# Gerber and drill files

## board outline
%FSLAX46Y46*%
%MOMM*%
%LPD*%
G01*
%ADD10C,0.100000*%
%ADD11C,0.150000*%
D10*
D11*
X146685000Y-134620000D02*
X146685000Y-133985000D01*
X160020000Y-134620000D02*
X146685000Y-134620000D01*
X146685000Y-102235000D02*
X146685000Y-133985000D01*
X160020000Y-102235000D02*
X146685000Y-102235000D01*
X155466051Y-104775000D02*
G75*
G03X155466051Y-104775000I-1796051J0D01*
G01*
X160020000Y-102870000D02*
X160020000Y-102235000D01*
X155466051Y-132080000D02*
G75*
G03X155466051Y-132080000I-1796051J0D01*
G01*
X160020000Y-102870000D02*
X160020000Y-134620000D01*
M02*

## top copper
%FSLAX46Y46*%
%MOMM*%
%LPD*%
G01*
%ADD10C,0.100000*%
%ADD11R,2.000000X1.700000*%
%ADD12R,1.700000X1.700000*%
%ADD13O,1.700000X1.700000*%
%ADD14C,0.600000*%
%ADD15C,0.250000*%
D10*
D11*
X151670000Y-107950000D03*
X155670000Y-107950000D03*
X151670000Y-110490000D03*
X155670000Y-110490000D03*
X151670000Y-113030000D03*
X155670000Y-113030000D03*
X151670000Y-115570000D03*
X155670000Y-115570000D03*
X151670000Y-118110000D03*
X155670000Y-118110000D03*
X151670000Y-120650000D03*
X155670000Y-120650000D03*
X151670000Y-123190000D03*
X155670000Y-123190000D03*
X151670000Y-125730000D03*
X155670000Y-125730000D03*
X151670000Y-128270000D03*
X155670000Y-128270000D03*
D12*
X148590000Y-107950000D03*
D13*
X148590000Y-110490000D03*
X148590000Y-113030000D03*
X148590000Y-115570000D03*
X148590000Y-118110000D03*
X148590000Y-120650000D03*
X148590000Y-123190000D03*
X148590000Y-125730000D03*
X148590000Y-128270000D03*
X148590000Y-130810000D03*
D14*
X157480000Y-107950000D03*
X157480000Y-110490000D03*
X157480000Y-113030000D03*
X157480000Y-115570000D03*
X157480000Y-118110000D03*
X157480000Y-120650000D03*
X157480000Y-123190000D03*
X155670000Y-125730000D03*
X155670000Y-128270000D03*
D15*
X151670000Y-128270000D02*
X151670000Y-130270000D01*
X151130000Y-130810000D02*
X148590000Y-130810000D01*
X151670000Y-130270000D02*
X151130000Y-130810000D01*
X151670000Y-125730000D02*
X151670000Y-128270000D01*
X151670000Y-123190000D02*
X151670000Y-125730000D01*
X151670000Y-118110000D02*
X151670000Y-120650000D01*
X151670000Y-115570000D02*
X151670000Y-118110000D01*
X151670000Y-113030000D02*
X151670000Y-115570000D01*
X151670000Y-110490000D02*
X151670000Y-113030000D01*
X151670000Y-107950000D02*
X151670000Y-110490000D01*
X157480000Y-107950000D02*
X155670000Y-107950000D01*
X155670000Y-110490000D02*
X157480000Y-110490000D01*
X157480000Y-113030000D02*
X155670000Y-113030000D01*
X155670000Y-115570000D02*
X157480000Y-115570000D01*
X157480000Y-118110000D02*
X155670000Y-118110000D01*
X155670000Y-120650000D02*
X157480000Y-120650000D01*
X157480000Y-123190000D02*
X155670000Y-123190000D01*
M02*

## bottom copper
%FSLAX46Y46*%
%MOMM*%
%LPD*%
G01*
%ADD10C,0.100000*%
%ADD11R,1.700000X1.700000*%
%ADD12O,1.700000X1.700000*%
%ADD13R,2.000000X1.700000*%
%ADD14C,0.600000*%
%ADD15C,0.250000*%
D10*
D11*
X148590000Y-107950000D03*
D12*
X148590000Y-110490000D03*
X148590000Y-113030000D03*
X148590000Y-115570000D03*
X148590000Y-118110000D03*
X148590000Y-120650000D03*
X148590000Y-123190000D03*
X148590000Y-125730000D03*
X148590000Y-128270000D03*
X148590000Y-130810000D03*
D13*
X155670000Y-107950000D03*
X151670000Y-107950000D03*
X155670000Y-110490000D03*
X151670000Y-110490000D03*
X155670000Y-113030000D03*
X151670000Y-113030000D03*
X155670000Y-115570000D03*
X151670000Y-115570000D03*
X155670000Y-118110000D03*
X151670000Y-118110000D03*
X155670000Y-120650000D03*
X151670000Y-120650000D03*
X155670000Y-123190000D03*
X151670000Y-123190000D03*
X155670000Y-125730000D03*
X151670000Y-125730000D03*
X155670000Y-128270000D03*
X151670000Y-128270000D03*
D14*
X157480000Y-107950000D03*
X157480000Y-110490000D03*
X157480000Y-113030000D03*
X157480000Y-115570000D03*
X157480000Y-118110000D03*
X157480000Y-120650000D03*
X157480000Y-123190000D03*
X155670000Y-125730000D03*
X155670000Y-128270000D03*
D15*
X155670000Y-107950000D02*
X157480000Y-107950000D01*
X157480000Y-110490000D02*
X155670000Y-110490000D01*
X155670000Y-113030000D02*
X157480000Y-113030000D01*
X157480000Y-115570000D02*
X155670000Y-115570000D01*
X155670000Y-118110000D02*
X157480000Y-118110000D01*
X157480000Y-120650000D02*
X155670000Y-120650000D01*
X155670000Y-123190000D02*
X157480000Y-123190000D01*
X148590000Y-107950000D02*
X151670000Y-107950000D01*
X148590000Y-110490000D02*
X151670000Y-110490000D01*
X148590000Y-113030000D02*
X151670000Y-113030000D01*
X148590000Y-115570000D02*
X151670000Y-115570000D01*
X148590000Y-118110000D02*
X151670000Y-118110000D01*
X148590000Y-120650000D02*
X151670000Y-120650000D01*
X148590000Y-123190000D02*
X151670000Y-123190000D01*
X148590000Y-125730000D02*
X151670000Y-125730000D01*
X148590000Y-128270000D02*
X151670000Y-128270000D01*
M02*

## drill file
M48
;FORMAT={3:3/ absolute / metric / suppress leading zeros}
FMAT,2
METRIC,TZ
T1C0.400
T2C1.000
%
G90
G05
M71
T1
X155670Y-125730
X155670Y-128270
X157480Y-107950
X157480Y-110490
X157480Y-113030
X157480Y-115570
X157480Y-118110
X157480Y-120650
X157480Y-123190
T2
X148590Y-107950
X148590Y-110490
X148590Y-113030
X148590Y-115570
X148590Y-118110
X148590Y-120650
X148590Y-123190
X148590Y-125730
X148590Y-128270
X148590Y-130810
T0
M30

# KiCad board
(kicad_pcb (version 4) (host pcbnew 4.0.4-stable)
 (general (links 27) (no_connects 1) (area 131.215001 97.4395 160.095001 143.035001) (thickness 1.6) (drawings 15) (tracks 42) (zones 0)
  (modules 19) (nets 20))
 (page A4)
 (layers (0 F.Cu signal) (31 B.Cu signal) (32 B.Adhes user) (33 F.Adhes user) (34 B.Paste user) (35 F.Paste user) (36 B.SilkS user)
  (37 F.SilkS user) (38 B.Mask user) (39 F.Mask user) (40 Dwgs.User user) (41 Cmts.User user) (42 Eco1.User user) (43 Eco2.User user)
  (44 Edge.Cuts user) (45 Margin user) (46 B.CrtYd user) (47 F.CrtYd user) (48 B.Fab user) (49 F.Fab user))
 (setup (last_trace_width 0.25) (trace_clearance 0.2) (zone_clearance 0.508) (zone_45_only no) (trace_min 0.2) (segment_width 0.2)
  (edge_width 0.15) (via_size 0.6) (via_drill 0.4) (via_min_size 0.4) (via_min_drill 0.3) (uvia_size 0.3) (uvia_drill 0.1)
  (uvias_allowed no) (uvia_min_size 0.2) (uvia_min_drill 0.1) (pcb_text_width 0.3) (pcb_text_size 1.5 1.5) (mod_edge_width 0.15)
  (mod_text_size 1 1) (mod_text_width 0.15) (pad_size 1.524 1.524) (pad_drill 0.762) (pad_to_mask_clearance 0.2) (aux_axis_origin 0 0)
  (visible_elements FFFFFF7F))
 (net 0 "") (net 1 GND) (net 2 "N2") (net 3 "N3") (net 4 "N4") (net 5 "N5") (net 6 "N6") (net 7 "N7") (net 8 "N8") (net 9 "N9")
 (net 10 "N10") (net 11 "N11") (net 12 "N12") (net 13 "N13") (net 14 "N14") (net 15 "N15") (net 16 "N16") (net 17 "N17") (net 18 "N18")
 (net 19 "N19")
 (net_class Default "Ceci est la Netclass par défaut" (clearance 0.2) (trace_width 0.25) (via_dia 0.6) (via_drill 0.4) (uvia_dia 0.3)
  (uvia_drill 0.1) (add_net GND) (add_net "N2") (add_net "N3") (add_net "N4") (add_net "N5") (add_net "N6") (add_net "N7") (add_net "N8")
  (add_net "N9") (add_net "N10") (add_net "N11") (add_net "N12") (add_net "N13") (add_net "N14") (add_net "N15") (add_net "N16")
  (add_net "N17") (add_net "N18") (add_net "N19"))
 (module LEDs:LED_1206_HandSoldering (layer F.Cu) (at 153.67 107.95)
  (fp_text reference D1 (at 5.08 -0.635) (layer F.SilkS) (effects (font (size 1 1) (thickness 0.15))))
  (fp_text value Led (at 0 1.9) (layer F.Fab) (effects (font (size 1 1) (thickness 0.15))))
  (pad 1 smd rect (at -2 0) (size 2 1.7) (layers F.Cu F.Paste F.Mask) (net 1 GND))
  (pad 2 smd rect (at 2 0) (size 2 1.7) (layers F.Cu F.Paste F.Mask) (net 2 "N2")))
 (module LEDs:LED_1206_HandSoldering (layer F.Cu) (at 153.67 110.49)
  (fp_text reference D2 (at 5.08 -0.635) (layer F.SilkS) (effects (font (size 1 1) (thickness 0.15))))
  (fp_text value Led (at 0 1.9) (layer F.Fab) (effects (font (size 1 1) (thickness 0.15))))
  (pad 1 smd rect (at -2 0) (size 2 1.7) (layers F.Cu F.Paste F.Mask) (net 1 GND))
  (pad 2 smd rect (at 2 0) (size 2 1.7) (layers F.Cu F.Paste F.Mask) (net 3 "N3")))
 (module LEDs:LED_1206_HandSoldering (layer F.Cu) (at 153.67 113.03)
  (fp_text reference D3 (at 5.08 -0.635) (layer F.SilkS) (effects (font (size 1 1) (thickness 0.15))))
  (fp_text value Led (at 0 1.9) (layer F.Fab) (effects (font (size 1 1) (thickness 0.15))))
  (pad 1 smd rect (at -2 0) (size 2 1.7) (layers F.Cu F.Paste F.Mask) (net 1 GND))
  (pad 2 smd rect (at 2 0) (size 2 1.7) (layers F.Cu F.Paste F.Mask) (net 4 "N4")))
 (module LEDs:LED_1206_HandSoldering (layer F.Cu) (at 153.67 115.57)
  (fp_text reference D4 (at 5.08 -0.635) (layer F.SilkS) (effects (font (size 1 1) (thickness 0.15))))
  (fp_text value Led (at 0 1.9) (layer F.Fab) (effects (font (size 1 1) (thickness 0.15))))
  (pad 1 smd rect (at -2 0) (size 2 1.7) (layers F.Cu F.Paste F.Mask) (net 1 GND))
  (pad 2 smd rect (at 2 0) (size 2 1.7) (layers F.Cu F.Paste F.Mask) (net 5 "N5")))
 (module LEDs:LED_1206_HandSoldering (layer F.Cu) (at 153.67 118.11)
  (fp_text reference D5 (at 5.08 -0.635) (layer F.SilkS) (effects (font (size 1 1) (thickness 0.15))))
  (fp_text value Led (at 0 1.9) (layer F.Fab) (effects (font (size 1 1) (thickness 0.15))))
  (pad 1 smd rect (at -2 0) (size 2 1.7) (layers F.Cu F.Paste F.Mask) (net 1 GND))
  (pad 2 smd rect (at 2 0) (size 2 1.7) (layers F.Cu F.Paste F.Mask) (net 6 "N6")))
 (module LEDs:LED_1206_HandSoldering (layer F.Cu) (at 153.67 120.65)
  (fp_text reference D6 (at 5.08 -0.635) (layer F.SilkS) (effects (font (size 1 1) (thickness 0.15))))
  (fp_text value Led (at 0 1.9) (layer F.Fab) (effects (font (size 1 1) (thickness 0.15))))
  (pad 1 smd rect (at -2 0) (size 2 1.7) (layers F.Cu F.Paste F.Mask) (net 1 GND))
  (pad 2 smd rect (at 2 0) (size 2 1.7) (layers F.Cu F.Paste F.Mask) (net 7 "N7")))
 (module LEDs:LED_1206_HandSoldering (layer F.Cu) (at 153.67 123.19)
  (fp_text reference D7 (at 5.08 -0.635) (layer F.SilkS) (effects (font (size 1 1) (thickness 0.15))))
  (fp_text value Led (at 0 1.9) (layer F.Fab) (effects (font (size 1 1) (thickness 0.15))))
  (pad 1 smd rect (at -2 0) (size 2 1.7) (layers F.Cu F.Paste F.Mask) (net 1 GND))
  (pad 2 smd rect (at 2 0) (size 2 1.7) (layers F.Cu F.Paste F.Mask) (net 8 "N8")))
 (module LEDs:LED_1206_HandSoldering (layer F.Cu) (at 153.67 125.73)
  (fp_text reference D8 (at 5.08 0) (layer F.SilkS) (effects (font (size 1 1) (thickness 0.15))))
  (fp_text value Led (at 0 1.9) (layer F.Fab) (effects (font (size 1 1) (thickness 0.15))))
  (pad 1 smd rect (at -2 0) (size 2 1.7) (layers F.Cu F.Paste F.Mask) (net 1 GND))
  (pad 2 smd rect (at 2 0) (size 2 1.7) (layers F.Cu F.Paste F.Mask) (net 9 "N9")))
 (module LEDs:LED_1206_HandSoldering (layer F.Cu) (at 153.67 128.27)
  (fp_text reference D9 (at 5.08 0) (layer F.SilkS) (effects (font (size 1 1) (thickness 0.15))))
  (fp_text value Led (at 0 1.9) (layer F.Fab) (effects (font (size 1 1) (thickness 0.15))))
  (pad 1 smd rect (at -2 0) (size 2 1.7) (layers F.Cu F.Paste F.Mask) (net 1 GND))
  (pad 2 smd rect (at 2 0) (size 2 1.7) (layers F.Cu F.Paste F.Mask) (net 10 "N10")))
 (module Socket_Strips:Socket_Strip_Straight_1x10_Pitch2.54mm (layer F.Cu) (at 148.59 107.95)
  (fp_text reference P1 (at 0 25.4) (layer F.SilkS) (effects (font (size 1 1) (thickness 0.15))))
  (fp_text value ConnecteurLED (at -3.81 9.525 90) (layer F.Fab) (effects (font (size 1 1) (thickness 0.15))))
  (pad 1 thru_hole rect (at 0 0) (size 1.7 1.7) (drill 1) (layers *.Cu *.Mask) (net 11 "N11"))
  (pad 2 thru_hole oval (at 0 2.54) (size 1.7 1.7) (drill 1) (layers *.Cu *.Mask) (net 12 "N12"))
  (pad 3 thru_hole oval (at 0 5.08) (size 1.7 1.7) (drill 1) (layers *.Cu *.Mask) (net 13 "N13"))
  (pad 4 thru_hole oval (at 0 7.62) (size 1.7 1.7) (drill 1) (layers *.Cu *.Mask) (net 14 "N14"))
  (pad 5 thru_hole oval (at 0 10.16) (size 1.7 1.7) (drill 1) (layers *.Cu *.Mask) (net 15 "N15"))
  (pad 6 thru_hole oval (at 0 12.7) (size 1.7 1.7) (drill 1) (layers *.Cu *.Mask) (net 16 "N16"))
  (pad 7 thru_hole oval (at 0 15.24) (size 1.7 1.7) (drill 1) (layers *.Cu *.Mask) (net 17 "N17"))
  (pad 8 thru_hole oval (at 0 17.78) (size 1.7 1.7) (drill 1) (layers *.Cu *.Mask) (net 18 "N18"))
  (pad 9 thru_hole oval (at 0 20.32) (size 1.7 1.7) (drill 1) (layers *.Cu *.Mask) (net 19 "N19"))
  (pad 10 thru_hole oval (at 0 22.86) (size 1.7 1.7) (drill 1) (layers *.Cu *.Mask) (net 1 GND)))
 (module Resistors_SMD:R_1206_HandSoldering (layer B.Cu) (at 153.67 107.95 180)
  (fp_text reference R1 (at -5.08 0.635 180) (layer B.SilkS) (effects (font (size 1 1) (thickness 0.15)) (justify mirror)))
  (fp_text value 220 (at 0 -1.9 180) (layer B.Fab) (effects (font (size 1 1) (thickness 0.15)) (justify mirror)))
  (pad 1 smd rect (at -2 0 180) (size 2 1.7) (layers B.Cu B.Paste B.Mask) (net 2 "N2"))
  (pad 2 smd rect (at 2 0 180) (size 2 1.7) (layers B.Cu B.Paste B.Mask) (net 11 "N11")))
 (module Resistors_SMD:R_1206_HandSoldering (layer B.Cu) (at 153.67 110.49 180)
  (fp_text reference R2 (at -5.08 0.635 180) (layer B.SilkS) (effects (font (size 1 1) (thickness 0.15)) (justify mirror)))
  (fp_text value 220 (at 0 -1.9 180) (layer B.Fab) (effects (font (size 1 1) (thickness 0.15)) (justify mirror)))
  (pad 1 smd rect (at -2 0 180) (size 2 1.7) (layers B.Cu B.Paste B.Mask) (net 3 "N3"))
  (pad 2 smd rect (at 2 0 180) (size 2 1.7) (layers B.Cu B.Paste B.Mask) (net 12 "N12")))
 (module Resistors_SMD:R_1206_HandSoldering (layer B.Cu) (at 153.67 113.03 180)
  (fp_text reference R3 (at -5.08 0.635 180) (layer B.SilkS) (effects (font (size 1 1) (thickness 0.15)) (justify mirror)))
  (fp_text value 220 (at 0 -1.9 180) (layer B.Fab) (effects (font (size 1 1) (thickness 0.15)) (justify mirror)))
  (pad 1 smd rect (at -2 0 180) (size 2 1.7) (layers B.Cu B.Paste B.Mask) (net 4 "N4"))
  (pad 2 smd rect (at 2 0 180) (size 2 1.7) (layers B.Cu B.Paste B.Mask) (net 13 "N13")))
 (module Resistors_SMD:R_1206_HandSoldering (layer B.Cu) (at 153.67 115.57 180)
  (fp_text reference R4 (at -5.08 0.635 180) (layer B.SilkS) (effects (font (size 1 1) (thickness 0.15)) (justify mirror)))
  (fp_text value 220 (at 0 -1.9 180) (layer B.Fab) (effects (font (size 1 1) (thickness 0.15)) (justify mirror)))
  (pad 1 smd rect (at -2 0 180) (size 2 1.7) (layers B.Cu B.Paste B.Mask) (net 5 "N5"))
  (pad 2 smd rect (at 2 0 180) (size 2 1.7) (layers B.Cu B.Paste B.Mask) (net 14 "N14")))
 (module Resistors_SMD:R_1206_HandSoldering (layer B.Cu) (at 153.67 118.11 180)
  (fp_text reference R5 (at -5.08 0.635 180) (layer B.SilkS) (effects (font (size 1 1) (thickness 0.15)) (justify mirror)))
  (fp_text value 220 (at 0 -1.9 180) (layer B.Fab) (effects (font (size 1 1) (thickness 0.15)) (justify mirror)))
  (pad 1 smd rect (at -2 0 180) (size 2 1.7) (layers B.Cu B.Paste B.Mask) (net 6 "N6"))
  (pad 2 smd rect (at 2 0 180) (size 2 1.7) (layers B.Cu B.Paste B.Mask) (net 15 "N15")))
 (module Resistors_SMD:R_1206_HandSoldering (layer B.Cu) (at 153.67 120.65 180)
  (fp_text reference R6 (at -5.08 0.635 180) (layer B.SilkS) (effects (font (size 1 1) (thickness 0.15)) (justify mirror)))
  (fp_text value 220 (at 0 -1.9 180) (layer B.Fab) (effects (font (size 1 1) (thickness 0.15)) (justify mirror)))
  (pad 1 smd rect (at -2 0 180) (size 2 1.7) (layers B.Cu B.Paste B.Mask) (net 7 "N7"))
  (pad 2 smd rect (at 2 0 180) (size 2 1.7) (layers B.Cu B.Paste B.Mask) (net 16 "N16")))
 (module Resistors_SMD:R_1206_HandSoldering (layer B.Cu) (at 153.67 123.19 180)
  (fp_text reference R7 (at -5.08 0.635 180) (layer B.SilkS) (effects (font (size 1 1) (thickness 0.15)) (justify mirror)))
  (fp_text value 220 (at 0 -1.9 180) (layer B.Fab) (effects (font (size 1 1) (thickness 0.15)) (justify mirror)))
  (pad 1 smd rect (at -2 0 180) (size 2 1.7) (layers B.Cu B.Paste B.Mask) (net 8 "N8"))
  (pad 2 smd rect (at 2 0 180) (size 2 1.7) (layers B.Cu B.Paste B.Mask) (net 17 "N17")))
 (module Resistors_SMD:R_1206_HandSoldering (layer B.Cu) (at 153.67 125.73 180)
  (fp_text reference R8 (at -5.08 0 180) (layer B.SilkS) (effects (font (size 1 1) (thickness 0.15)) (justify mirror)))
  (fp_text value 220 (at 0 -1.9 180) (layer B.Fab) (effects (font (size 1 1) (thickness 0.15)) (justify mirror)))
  (pad 1 smd rect (at -2 0 180) (size 2 1.7) (layers B.Cu B.Paste B.Mask) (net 9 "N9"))
  (pad 2 smd rect (at 2 0 180) (size 2 1.7) (layers B.Cu B.Paste B.Mask) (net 18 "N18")))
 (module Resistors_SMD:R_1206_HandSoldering (layer B.Cu) (at 153.67 128.27 180)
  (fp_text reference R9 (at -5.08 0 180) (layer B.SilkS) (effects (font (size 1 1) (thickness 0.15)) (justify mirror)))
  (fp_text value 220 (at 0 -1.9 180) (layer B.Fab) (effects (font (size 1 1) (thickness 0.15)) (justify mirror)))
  (pad 1 smd rect (at -2 0 180) (size 2 1.7) (layers B.Cu B.Paste B.Mask) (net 10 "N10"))
  (pad 2 smd rect (at 2 0 180) (size 2 1.7) (layers B.Cu B.Paste B.Mask) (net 19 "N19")))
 (gr_line (start 146.685 134.62) (end 146.685 133.985) (angle 90) (layer Edge.Cuts) (width 0.15))
 (gr_line (start 160.02 134.62) (end 146.685 134.62) (angle 90) (layer Edge.Cuts) (width 0.15))
 (gr_line (start 146.685 102.235) (end 146.685 133.985) (angle 90) (layer Edge.Cuts) (width 0.15))
 (gr_line (start 160.02 102.235) (end 146.685 102.235) (angle 90) (layer Edge.Cuts) (width 0.15))
 (gr_circle (center 153.67 104.775) (end 154.94 103.505) (layer Edge.Cuts) (width 0.15))
 (gr_line (start 160.02 102.87) (end 160.02 102.235) (angle 90) (layer Edge.Cuts) (width 0.15))
 (gr_circle (center 153.67 132.08) (end 154.94 130.81) (layer Edge.Cuts) (width 0.15))
 (gr_line (start 160.02 102.87) (end 160.02 134.62) (angle 90) (layer Edge.Cuts) (width 0.15))
 (segment (start 151.67 128.27) (end 151.67 130.27) (width 0.25) (layer F.Cu) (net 1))
 (segment (start 151.13 130.81) (end 148.59 130.81) (width 0.25) (layer F.Cu) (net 1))
 (segment (start 151.67 130.27) (end 151.13 130.81) (width 0.25) (layer F.Cu) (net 1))
 (segment (start 151.67 125.73) (end 151.67 128.27) (width 0.25) (layer F.Cu) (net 1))
 (segment (start 151.67 123.19) (end 151.67 125.73) (width 0.25) (layer F.Cu) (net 1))
 (segment (start 151.67 118.11) (end 151.67 120.65) (width 0.25) (layer F.Cu) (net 1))
 (segment (start 151.67 115.57) (end 151.67 118.11) (width 0.25) (layer F.Cu) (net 1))
 (segment (start 151.67 113.03) (end 151.67 115.57) (width 0.25) (layer F.Cu) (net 1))
 (segment (start 151.67 110.49) (end 151.67 113.03) (width 0.25) (layer F.Cu) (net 1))
 (segment (start 151.67 107.95) (end 151.67 110.49) (width 0.25) (layer F.Cu) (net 1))
 (segment (start 155.67 107.95) (end 157.48 107.95) (width 0.25) (layer B.Cu) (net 2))
 (segment (start 157.48 107.95) (end 155.67 107.95) (width 0.25) (layer F.Cu) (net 2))
 (via (at 157.48 107.95) (size 0.6) (drill 0.4) (layers F.Cu B.Cu) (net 2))
 (segment (start 155.67 110.49) (end 157.48 110.49) (width 0.25) (layer F.Cu) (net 3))
 (segment (start 157.48 110.49) (end 155.67 110.49) (width 0.25) (layer B.Cu) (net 3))
 (via (at 157.48 110.49) (size 0.6) (drill 0.4) (layers F.Cu B.Cu) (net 3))
 (segment (start 155.67 113.03) (end 157.48 113.03) (width 0.25) (layer B.Cu) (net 4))
 (segment (start 157.48 113.03) (end 155.67 113.03) (width 0.25) (layer F.Cu) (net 4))
 (via (at 157.48 113.03) (size 0.6) (drill 0.4) (layers F.Cu B.Cu) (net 4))
 (segment (start 155.67 115.57) (end 157.48 115.57) (width 0.25) (layer F.Cu) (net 5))
 (segment (start 157.48 115.57) (end 155.67 115.57) (width 0.25) (layer B.Cu) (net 5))
 (via (at 157.48 115.57) (size 0.6) (drill 0.4) (layers F.Cu B.Cu) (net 5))
 (segment (start 155.67 118.11) (end 157.48 118.11) (width 0.25) (layer B.Cu) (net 6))
 (segment (start 157.48 118.11) (end 155.67 118.11) (width 0.25) (layer F.Cu) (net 6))
 (via (at 157.48 118.11) (size 0.6) (drill 0.4) (layers F.Cu B.Cu) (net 6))
 (segment (start 155.67 120.65) (end 157.48 120.65) (width 0.25) (layer F.Cu) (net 7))
 (segment (start 157.48 120.65) (end 155.67 120.65) (width 0.25) (layer B.Cu) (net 7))
 (via (at 157.48 120.65) (size 0.6) (drill 0.4) (layers F.Cu B.Cu) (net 7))
 (segment (start 155.67 123.19) (end 157.48 123.19) (width 0.25) (layer B.Cu) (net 8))
 (segment (start 157.48 123.19) (end 155.67 123.19) (width 0.25) (layer F.Cu) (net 8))
 (via (at 157.48 123.19) (size 0.6) (drill 0.4) (layers F.Cu B.Cu) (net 8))
 (via (at 155.67 125.73) (size 0.6) (drill 0.4) (layers F.Cu B.Cu) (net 9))
 (via (at 155.67 128.27) (size 0.6) (drill 0.4) (layers F.Cu B.Cu) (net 10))
 (segment (start 148.59 107.95) (end 151.67 107.95) (width 0.25) (layer B.Cu) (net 11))
 (segment (start 148.59 110.49) (end 151.67 110.49) (width 0.25) (layer B.Cu) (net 12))
 (segment (start 148.59 113.03) (end 151.67 113.03) (width 0.25) (layer B.Cu) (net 13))
 (segment (start 148.59 115.57) (end 151.67 115.57) (width 0.25) (layer B.Cu) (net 14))
 (segment (start 148.59 118.11) (end 151.67 118.11) (width 0.25) (layer B.Cu) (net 15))
 (segment (start 148.59 120.65) (end 151.67 120.65) (width 0.25) (layer B.Cu) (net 16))
 (segment (start 148.59 123.19) (end 151.67 123.19) (width 0.25) (layer B.Cu) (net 17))
 (segment (start 148.59 125.73) (end 151.67 125.73) (width 0.25) (layer B.Cu) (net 18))
 (segment (start 148.59 128.27) (end 151.67 128.27) (width 0.25) (layer B.Cu) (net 19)))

